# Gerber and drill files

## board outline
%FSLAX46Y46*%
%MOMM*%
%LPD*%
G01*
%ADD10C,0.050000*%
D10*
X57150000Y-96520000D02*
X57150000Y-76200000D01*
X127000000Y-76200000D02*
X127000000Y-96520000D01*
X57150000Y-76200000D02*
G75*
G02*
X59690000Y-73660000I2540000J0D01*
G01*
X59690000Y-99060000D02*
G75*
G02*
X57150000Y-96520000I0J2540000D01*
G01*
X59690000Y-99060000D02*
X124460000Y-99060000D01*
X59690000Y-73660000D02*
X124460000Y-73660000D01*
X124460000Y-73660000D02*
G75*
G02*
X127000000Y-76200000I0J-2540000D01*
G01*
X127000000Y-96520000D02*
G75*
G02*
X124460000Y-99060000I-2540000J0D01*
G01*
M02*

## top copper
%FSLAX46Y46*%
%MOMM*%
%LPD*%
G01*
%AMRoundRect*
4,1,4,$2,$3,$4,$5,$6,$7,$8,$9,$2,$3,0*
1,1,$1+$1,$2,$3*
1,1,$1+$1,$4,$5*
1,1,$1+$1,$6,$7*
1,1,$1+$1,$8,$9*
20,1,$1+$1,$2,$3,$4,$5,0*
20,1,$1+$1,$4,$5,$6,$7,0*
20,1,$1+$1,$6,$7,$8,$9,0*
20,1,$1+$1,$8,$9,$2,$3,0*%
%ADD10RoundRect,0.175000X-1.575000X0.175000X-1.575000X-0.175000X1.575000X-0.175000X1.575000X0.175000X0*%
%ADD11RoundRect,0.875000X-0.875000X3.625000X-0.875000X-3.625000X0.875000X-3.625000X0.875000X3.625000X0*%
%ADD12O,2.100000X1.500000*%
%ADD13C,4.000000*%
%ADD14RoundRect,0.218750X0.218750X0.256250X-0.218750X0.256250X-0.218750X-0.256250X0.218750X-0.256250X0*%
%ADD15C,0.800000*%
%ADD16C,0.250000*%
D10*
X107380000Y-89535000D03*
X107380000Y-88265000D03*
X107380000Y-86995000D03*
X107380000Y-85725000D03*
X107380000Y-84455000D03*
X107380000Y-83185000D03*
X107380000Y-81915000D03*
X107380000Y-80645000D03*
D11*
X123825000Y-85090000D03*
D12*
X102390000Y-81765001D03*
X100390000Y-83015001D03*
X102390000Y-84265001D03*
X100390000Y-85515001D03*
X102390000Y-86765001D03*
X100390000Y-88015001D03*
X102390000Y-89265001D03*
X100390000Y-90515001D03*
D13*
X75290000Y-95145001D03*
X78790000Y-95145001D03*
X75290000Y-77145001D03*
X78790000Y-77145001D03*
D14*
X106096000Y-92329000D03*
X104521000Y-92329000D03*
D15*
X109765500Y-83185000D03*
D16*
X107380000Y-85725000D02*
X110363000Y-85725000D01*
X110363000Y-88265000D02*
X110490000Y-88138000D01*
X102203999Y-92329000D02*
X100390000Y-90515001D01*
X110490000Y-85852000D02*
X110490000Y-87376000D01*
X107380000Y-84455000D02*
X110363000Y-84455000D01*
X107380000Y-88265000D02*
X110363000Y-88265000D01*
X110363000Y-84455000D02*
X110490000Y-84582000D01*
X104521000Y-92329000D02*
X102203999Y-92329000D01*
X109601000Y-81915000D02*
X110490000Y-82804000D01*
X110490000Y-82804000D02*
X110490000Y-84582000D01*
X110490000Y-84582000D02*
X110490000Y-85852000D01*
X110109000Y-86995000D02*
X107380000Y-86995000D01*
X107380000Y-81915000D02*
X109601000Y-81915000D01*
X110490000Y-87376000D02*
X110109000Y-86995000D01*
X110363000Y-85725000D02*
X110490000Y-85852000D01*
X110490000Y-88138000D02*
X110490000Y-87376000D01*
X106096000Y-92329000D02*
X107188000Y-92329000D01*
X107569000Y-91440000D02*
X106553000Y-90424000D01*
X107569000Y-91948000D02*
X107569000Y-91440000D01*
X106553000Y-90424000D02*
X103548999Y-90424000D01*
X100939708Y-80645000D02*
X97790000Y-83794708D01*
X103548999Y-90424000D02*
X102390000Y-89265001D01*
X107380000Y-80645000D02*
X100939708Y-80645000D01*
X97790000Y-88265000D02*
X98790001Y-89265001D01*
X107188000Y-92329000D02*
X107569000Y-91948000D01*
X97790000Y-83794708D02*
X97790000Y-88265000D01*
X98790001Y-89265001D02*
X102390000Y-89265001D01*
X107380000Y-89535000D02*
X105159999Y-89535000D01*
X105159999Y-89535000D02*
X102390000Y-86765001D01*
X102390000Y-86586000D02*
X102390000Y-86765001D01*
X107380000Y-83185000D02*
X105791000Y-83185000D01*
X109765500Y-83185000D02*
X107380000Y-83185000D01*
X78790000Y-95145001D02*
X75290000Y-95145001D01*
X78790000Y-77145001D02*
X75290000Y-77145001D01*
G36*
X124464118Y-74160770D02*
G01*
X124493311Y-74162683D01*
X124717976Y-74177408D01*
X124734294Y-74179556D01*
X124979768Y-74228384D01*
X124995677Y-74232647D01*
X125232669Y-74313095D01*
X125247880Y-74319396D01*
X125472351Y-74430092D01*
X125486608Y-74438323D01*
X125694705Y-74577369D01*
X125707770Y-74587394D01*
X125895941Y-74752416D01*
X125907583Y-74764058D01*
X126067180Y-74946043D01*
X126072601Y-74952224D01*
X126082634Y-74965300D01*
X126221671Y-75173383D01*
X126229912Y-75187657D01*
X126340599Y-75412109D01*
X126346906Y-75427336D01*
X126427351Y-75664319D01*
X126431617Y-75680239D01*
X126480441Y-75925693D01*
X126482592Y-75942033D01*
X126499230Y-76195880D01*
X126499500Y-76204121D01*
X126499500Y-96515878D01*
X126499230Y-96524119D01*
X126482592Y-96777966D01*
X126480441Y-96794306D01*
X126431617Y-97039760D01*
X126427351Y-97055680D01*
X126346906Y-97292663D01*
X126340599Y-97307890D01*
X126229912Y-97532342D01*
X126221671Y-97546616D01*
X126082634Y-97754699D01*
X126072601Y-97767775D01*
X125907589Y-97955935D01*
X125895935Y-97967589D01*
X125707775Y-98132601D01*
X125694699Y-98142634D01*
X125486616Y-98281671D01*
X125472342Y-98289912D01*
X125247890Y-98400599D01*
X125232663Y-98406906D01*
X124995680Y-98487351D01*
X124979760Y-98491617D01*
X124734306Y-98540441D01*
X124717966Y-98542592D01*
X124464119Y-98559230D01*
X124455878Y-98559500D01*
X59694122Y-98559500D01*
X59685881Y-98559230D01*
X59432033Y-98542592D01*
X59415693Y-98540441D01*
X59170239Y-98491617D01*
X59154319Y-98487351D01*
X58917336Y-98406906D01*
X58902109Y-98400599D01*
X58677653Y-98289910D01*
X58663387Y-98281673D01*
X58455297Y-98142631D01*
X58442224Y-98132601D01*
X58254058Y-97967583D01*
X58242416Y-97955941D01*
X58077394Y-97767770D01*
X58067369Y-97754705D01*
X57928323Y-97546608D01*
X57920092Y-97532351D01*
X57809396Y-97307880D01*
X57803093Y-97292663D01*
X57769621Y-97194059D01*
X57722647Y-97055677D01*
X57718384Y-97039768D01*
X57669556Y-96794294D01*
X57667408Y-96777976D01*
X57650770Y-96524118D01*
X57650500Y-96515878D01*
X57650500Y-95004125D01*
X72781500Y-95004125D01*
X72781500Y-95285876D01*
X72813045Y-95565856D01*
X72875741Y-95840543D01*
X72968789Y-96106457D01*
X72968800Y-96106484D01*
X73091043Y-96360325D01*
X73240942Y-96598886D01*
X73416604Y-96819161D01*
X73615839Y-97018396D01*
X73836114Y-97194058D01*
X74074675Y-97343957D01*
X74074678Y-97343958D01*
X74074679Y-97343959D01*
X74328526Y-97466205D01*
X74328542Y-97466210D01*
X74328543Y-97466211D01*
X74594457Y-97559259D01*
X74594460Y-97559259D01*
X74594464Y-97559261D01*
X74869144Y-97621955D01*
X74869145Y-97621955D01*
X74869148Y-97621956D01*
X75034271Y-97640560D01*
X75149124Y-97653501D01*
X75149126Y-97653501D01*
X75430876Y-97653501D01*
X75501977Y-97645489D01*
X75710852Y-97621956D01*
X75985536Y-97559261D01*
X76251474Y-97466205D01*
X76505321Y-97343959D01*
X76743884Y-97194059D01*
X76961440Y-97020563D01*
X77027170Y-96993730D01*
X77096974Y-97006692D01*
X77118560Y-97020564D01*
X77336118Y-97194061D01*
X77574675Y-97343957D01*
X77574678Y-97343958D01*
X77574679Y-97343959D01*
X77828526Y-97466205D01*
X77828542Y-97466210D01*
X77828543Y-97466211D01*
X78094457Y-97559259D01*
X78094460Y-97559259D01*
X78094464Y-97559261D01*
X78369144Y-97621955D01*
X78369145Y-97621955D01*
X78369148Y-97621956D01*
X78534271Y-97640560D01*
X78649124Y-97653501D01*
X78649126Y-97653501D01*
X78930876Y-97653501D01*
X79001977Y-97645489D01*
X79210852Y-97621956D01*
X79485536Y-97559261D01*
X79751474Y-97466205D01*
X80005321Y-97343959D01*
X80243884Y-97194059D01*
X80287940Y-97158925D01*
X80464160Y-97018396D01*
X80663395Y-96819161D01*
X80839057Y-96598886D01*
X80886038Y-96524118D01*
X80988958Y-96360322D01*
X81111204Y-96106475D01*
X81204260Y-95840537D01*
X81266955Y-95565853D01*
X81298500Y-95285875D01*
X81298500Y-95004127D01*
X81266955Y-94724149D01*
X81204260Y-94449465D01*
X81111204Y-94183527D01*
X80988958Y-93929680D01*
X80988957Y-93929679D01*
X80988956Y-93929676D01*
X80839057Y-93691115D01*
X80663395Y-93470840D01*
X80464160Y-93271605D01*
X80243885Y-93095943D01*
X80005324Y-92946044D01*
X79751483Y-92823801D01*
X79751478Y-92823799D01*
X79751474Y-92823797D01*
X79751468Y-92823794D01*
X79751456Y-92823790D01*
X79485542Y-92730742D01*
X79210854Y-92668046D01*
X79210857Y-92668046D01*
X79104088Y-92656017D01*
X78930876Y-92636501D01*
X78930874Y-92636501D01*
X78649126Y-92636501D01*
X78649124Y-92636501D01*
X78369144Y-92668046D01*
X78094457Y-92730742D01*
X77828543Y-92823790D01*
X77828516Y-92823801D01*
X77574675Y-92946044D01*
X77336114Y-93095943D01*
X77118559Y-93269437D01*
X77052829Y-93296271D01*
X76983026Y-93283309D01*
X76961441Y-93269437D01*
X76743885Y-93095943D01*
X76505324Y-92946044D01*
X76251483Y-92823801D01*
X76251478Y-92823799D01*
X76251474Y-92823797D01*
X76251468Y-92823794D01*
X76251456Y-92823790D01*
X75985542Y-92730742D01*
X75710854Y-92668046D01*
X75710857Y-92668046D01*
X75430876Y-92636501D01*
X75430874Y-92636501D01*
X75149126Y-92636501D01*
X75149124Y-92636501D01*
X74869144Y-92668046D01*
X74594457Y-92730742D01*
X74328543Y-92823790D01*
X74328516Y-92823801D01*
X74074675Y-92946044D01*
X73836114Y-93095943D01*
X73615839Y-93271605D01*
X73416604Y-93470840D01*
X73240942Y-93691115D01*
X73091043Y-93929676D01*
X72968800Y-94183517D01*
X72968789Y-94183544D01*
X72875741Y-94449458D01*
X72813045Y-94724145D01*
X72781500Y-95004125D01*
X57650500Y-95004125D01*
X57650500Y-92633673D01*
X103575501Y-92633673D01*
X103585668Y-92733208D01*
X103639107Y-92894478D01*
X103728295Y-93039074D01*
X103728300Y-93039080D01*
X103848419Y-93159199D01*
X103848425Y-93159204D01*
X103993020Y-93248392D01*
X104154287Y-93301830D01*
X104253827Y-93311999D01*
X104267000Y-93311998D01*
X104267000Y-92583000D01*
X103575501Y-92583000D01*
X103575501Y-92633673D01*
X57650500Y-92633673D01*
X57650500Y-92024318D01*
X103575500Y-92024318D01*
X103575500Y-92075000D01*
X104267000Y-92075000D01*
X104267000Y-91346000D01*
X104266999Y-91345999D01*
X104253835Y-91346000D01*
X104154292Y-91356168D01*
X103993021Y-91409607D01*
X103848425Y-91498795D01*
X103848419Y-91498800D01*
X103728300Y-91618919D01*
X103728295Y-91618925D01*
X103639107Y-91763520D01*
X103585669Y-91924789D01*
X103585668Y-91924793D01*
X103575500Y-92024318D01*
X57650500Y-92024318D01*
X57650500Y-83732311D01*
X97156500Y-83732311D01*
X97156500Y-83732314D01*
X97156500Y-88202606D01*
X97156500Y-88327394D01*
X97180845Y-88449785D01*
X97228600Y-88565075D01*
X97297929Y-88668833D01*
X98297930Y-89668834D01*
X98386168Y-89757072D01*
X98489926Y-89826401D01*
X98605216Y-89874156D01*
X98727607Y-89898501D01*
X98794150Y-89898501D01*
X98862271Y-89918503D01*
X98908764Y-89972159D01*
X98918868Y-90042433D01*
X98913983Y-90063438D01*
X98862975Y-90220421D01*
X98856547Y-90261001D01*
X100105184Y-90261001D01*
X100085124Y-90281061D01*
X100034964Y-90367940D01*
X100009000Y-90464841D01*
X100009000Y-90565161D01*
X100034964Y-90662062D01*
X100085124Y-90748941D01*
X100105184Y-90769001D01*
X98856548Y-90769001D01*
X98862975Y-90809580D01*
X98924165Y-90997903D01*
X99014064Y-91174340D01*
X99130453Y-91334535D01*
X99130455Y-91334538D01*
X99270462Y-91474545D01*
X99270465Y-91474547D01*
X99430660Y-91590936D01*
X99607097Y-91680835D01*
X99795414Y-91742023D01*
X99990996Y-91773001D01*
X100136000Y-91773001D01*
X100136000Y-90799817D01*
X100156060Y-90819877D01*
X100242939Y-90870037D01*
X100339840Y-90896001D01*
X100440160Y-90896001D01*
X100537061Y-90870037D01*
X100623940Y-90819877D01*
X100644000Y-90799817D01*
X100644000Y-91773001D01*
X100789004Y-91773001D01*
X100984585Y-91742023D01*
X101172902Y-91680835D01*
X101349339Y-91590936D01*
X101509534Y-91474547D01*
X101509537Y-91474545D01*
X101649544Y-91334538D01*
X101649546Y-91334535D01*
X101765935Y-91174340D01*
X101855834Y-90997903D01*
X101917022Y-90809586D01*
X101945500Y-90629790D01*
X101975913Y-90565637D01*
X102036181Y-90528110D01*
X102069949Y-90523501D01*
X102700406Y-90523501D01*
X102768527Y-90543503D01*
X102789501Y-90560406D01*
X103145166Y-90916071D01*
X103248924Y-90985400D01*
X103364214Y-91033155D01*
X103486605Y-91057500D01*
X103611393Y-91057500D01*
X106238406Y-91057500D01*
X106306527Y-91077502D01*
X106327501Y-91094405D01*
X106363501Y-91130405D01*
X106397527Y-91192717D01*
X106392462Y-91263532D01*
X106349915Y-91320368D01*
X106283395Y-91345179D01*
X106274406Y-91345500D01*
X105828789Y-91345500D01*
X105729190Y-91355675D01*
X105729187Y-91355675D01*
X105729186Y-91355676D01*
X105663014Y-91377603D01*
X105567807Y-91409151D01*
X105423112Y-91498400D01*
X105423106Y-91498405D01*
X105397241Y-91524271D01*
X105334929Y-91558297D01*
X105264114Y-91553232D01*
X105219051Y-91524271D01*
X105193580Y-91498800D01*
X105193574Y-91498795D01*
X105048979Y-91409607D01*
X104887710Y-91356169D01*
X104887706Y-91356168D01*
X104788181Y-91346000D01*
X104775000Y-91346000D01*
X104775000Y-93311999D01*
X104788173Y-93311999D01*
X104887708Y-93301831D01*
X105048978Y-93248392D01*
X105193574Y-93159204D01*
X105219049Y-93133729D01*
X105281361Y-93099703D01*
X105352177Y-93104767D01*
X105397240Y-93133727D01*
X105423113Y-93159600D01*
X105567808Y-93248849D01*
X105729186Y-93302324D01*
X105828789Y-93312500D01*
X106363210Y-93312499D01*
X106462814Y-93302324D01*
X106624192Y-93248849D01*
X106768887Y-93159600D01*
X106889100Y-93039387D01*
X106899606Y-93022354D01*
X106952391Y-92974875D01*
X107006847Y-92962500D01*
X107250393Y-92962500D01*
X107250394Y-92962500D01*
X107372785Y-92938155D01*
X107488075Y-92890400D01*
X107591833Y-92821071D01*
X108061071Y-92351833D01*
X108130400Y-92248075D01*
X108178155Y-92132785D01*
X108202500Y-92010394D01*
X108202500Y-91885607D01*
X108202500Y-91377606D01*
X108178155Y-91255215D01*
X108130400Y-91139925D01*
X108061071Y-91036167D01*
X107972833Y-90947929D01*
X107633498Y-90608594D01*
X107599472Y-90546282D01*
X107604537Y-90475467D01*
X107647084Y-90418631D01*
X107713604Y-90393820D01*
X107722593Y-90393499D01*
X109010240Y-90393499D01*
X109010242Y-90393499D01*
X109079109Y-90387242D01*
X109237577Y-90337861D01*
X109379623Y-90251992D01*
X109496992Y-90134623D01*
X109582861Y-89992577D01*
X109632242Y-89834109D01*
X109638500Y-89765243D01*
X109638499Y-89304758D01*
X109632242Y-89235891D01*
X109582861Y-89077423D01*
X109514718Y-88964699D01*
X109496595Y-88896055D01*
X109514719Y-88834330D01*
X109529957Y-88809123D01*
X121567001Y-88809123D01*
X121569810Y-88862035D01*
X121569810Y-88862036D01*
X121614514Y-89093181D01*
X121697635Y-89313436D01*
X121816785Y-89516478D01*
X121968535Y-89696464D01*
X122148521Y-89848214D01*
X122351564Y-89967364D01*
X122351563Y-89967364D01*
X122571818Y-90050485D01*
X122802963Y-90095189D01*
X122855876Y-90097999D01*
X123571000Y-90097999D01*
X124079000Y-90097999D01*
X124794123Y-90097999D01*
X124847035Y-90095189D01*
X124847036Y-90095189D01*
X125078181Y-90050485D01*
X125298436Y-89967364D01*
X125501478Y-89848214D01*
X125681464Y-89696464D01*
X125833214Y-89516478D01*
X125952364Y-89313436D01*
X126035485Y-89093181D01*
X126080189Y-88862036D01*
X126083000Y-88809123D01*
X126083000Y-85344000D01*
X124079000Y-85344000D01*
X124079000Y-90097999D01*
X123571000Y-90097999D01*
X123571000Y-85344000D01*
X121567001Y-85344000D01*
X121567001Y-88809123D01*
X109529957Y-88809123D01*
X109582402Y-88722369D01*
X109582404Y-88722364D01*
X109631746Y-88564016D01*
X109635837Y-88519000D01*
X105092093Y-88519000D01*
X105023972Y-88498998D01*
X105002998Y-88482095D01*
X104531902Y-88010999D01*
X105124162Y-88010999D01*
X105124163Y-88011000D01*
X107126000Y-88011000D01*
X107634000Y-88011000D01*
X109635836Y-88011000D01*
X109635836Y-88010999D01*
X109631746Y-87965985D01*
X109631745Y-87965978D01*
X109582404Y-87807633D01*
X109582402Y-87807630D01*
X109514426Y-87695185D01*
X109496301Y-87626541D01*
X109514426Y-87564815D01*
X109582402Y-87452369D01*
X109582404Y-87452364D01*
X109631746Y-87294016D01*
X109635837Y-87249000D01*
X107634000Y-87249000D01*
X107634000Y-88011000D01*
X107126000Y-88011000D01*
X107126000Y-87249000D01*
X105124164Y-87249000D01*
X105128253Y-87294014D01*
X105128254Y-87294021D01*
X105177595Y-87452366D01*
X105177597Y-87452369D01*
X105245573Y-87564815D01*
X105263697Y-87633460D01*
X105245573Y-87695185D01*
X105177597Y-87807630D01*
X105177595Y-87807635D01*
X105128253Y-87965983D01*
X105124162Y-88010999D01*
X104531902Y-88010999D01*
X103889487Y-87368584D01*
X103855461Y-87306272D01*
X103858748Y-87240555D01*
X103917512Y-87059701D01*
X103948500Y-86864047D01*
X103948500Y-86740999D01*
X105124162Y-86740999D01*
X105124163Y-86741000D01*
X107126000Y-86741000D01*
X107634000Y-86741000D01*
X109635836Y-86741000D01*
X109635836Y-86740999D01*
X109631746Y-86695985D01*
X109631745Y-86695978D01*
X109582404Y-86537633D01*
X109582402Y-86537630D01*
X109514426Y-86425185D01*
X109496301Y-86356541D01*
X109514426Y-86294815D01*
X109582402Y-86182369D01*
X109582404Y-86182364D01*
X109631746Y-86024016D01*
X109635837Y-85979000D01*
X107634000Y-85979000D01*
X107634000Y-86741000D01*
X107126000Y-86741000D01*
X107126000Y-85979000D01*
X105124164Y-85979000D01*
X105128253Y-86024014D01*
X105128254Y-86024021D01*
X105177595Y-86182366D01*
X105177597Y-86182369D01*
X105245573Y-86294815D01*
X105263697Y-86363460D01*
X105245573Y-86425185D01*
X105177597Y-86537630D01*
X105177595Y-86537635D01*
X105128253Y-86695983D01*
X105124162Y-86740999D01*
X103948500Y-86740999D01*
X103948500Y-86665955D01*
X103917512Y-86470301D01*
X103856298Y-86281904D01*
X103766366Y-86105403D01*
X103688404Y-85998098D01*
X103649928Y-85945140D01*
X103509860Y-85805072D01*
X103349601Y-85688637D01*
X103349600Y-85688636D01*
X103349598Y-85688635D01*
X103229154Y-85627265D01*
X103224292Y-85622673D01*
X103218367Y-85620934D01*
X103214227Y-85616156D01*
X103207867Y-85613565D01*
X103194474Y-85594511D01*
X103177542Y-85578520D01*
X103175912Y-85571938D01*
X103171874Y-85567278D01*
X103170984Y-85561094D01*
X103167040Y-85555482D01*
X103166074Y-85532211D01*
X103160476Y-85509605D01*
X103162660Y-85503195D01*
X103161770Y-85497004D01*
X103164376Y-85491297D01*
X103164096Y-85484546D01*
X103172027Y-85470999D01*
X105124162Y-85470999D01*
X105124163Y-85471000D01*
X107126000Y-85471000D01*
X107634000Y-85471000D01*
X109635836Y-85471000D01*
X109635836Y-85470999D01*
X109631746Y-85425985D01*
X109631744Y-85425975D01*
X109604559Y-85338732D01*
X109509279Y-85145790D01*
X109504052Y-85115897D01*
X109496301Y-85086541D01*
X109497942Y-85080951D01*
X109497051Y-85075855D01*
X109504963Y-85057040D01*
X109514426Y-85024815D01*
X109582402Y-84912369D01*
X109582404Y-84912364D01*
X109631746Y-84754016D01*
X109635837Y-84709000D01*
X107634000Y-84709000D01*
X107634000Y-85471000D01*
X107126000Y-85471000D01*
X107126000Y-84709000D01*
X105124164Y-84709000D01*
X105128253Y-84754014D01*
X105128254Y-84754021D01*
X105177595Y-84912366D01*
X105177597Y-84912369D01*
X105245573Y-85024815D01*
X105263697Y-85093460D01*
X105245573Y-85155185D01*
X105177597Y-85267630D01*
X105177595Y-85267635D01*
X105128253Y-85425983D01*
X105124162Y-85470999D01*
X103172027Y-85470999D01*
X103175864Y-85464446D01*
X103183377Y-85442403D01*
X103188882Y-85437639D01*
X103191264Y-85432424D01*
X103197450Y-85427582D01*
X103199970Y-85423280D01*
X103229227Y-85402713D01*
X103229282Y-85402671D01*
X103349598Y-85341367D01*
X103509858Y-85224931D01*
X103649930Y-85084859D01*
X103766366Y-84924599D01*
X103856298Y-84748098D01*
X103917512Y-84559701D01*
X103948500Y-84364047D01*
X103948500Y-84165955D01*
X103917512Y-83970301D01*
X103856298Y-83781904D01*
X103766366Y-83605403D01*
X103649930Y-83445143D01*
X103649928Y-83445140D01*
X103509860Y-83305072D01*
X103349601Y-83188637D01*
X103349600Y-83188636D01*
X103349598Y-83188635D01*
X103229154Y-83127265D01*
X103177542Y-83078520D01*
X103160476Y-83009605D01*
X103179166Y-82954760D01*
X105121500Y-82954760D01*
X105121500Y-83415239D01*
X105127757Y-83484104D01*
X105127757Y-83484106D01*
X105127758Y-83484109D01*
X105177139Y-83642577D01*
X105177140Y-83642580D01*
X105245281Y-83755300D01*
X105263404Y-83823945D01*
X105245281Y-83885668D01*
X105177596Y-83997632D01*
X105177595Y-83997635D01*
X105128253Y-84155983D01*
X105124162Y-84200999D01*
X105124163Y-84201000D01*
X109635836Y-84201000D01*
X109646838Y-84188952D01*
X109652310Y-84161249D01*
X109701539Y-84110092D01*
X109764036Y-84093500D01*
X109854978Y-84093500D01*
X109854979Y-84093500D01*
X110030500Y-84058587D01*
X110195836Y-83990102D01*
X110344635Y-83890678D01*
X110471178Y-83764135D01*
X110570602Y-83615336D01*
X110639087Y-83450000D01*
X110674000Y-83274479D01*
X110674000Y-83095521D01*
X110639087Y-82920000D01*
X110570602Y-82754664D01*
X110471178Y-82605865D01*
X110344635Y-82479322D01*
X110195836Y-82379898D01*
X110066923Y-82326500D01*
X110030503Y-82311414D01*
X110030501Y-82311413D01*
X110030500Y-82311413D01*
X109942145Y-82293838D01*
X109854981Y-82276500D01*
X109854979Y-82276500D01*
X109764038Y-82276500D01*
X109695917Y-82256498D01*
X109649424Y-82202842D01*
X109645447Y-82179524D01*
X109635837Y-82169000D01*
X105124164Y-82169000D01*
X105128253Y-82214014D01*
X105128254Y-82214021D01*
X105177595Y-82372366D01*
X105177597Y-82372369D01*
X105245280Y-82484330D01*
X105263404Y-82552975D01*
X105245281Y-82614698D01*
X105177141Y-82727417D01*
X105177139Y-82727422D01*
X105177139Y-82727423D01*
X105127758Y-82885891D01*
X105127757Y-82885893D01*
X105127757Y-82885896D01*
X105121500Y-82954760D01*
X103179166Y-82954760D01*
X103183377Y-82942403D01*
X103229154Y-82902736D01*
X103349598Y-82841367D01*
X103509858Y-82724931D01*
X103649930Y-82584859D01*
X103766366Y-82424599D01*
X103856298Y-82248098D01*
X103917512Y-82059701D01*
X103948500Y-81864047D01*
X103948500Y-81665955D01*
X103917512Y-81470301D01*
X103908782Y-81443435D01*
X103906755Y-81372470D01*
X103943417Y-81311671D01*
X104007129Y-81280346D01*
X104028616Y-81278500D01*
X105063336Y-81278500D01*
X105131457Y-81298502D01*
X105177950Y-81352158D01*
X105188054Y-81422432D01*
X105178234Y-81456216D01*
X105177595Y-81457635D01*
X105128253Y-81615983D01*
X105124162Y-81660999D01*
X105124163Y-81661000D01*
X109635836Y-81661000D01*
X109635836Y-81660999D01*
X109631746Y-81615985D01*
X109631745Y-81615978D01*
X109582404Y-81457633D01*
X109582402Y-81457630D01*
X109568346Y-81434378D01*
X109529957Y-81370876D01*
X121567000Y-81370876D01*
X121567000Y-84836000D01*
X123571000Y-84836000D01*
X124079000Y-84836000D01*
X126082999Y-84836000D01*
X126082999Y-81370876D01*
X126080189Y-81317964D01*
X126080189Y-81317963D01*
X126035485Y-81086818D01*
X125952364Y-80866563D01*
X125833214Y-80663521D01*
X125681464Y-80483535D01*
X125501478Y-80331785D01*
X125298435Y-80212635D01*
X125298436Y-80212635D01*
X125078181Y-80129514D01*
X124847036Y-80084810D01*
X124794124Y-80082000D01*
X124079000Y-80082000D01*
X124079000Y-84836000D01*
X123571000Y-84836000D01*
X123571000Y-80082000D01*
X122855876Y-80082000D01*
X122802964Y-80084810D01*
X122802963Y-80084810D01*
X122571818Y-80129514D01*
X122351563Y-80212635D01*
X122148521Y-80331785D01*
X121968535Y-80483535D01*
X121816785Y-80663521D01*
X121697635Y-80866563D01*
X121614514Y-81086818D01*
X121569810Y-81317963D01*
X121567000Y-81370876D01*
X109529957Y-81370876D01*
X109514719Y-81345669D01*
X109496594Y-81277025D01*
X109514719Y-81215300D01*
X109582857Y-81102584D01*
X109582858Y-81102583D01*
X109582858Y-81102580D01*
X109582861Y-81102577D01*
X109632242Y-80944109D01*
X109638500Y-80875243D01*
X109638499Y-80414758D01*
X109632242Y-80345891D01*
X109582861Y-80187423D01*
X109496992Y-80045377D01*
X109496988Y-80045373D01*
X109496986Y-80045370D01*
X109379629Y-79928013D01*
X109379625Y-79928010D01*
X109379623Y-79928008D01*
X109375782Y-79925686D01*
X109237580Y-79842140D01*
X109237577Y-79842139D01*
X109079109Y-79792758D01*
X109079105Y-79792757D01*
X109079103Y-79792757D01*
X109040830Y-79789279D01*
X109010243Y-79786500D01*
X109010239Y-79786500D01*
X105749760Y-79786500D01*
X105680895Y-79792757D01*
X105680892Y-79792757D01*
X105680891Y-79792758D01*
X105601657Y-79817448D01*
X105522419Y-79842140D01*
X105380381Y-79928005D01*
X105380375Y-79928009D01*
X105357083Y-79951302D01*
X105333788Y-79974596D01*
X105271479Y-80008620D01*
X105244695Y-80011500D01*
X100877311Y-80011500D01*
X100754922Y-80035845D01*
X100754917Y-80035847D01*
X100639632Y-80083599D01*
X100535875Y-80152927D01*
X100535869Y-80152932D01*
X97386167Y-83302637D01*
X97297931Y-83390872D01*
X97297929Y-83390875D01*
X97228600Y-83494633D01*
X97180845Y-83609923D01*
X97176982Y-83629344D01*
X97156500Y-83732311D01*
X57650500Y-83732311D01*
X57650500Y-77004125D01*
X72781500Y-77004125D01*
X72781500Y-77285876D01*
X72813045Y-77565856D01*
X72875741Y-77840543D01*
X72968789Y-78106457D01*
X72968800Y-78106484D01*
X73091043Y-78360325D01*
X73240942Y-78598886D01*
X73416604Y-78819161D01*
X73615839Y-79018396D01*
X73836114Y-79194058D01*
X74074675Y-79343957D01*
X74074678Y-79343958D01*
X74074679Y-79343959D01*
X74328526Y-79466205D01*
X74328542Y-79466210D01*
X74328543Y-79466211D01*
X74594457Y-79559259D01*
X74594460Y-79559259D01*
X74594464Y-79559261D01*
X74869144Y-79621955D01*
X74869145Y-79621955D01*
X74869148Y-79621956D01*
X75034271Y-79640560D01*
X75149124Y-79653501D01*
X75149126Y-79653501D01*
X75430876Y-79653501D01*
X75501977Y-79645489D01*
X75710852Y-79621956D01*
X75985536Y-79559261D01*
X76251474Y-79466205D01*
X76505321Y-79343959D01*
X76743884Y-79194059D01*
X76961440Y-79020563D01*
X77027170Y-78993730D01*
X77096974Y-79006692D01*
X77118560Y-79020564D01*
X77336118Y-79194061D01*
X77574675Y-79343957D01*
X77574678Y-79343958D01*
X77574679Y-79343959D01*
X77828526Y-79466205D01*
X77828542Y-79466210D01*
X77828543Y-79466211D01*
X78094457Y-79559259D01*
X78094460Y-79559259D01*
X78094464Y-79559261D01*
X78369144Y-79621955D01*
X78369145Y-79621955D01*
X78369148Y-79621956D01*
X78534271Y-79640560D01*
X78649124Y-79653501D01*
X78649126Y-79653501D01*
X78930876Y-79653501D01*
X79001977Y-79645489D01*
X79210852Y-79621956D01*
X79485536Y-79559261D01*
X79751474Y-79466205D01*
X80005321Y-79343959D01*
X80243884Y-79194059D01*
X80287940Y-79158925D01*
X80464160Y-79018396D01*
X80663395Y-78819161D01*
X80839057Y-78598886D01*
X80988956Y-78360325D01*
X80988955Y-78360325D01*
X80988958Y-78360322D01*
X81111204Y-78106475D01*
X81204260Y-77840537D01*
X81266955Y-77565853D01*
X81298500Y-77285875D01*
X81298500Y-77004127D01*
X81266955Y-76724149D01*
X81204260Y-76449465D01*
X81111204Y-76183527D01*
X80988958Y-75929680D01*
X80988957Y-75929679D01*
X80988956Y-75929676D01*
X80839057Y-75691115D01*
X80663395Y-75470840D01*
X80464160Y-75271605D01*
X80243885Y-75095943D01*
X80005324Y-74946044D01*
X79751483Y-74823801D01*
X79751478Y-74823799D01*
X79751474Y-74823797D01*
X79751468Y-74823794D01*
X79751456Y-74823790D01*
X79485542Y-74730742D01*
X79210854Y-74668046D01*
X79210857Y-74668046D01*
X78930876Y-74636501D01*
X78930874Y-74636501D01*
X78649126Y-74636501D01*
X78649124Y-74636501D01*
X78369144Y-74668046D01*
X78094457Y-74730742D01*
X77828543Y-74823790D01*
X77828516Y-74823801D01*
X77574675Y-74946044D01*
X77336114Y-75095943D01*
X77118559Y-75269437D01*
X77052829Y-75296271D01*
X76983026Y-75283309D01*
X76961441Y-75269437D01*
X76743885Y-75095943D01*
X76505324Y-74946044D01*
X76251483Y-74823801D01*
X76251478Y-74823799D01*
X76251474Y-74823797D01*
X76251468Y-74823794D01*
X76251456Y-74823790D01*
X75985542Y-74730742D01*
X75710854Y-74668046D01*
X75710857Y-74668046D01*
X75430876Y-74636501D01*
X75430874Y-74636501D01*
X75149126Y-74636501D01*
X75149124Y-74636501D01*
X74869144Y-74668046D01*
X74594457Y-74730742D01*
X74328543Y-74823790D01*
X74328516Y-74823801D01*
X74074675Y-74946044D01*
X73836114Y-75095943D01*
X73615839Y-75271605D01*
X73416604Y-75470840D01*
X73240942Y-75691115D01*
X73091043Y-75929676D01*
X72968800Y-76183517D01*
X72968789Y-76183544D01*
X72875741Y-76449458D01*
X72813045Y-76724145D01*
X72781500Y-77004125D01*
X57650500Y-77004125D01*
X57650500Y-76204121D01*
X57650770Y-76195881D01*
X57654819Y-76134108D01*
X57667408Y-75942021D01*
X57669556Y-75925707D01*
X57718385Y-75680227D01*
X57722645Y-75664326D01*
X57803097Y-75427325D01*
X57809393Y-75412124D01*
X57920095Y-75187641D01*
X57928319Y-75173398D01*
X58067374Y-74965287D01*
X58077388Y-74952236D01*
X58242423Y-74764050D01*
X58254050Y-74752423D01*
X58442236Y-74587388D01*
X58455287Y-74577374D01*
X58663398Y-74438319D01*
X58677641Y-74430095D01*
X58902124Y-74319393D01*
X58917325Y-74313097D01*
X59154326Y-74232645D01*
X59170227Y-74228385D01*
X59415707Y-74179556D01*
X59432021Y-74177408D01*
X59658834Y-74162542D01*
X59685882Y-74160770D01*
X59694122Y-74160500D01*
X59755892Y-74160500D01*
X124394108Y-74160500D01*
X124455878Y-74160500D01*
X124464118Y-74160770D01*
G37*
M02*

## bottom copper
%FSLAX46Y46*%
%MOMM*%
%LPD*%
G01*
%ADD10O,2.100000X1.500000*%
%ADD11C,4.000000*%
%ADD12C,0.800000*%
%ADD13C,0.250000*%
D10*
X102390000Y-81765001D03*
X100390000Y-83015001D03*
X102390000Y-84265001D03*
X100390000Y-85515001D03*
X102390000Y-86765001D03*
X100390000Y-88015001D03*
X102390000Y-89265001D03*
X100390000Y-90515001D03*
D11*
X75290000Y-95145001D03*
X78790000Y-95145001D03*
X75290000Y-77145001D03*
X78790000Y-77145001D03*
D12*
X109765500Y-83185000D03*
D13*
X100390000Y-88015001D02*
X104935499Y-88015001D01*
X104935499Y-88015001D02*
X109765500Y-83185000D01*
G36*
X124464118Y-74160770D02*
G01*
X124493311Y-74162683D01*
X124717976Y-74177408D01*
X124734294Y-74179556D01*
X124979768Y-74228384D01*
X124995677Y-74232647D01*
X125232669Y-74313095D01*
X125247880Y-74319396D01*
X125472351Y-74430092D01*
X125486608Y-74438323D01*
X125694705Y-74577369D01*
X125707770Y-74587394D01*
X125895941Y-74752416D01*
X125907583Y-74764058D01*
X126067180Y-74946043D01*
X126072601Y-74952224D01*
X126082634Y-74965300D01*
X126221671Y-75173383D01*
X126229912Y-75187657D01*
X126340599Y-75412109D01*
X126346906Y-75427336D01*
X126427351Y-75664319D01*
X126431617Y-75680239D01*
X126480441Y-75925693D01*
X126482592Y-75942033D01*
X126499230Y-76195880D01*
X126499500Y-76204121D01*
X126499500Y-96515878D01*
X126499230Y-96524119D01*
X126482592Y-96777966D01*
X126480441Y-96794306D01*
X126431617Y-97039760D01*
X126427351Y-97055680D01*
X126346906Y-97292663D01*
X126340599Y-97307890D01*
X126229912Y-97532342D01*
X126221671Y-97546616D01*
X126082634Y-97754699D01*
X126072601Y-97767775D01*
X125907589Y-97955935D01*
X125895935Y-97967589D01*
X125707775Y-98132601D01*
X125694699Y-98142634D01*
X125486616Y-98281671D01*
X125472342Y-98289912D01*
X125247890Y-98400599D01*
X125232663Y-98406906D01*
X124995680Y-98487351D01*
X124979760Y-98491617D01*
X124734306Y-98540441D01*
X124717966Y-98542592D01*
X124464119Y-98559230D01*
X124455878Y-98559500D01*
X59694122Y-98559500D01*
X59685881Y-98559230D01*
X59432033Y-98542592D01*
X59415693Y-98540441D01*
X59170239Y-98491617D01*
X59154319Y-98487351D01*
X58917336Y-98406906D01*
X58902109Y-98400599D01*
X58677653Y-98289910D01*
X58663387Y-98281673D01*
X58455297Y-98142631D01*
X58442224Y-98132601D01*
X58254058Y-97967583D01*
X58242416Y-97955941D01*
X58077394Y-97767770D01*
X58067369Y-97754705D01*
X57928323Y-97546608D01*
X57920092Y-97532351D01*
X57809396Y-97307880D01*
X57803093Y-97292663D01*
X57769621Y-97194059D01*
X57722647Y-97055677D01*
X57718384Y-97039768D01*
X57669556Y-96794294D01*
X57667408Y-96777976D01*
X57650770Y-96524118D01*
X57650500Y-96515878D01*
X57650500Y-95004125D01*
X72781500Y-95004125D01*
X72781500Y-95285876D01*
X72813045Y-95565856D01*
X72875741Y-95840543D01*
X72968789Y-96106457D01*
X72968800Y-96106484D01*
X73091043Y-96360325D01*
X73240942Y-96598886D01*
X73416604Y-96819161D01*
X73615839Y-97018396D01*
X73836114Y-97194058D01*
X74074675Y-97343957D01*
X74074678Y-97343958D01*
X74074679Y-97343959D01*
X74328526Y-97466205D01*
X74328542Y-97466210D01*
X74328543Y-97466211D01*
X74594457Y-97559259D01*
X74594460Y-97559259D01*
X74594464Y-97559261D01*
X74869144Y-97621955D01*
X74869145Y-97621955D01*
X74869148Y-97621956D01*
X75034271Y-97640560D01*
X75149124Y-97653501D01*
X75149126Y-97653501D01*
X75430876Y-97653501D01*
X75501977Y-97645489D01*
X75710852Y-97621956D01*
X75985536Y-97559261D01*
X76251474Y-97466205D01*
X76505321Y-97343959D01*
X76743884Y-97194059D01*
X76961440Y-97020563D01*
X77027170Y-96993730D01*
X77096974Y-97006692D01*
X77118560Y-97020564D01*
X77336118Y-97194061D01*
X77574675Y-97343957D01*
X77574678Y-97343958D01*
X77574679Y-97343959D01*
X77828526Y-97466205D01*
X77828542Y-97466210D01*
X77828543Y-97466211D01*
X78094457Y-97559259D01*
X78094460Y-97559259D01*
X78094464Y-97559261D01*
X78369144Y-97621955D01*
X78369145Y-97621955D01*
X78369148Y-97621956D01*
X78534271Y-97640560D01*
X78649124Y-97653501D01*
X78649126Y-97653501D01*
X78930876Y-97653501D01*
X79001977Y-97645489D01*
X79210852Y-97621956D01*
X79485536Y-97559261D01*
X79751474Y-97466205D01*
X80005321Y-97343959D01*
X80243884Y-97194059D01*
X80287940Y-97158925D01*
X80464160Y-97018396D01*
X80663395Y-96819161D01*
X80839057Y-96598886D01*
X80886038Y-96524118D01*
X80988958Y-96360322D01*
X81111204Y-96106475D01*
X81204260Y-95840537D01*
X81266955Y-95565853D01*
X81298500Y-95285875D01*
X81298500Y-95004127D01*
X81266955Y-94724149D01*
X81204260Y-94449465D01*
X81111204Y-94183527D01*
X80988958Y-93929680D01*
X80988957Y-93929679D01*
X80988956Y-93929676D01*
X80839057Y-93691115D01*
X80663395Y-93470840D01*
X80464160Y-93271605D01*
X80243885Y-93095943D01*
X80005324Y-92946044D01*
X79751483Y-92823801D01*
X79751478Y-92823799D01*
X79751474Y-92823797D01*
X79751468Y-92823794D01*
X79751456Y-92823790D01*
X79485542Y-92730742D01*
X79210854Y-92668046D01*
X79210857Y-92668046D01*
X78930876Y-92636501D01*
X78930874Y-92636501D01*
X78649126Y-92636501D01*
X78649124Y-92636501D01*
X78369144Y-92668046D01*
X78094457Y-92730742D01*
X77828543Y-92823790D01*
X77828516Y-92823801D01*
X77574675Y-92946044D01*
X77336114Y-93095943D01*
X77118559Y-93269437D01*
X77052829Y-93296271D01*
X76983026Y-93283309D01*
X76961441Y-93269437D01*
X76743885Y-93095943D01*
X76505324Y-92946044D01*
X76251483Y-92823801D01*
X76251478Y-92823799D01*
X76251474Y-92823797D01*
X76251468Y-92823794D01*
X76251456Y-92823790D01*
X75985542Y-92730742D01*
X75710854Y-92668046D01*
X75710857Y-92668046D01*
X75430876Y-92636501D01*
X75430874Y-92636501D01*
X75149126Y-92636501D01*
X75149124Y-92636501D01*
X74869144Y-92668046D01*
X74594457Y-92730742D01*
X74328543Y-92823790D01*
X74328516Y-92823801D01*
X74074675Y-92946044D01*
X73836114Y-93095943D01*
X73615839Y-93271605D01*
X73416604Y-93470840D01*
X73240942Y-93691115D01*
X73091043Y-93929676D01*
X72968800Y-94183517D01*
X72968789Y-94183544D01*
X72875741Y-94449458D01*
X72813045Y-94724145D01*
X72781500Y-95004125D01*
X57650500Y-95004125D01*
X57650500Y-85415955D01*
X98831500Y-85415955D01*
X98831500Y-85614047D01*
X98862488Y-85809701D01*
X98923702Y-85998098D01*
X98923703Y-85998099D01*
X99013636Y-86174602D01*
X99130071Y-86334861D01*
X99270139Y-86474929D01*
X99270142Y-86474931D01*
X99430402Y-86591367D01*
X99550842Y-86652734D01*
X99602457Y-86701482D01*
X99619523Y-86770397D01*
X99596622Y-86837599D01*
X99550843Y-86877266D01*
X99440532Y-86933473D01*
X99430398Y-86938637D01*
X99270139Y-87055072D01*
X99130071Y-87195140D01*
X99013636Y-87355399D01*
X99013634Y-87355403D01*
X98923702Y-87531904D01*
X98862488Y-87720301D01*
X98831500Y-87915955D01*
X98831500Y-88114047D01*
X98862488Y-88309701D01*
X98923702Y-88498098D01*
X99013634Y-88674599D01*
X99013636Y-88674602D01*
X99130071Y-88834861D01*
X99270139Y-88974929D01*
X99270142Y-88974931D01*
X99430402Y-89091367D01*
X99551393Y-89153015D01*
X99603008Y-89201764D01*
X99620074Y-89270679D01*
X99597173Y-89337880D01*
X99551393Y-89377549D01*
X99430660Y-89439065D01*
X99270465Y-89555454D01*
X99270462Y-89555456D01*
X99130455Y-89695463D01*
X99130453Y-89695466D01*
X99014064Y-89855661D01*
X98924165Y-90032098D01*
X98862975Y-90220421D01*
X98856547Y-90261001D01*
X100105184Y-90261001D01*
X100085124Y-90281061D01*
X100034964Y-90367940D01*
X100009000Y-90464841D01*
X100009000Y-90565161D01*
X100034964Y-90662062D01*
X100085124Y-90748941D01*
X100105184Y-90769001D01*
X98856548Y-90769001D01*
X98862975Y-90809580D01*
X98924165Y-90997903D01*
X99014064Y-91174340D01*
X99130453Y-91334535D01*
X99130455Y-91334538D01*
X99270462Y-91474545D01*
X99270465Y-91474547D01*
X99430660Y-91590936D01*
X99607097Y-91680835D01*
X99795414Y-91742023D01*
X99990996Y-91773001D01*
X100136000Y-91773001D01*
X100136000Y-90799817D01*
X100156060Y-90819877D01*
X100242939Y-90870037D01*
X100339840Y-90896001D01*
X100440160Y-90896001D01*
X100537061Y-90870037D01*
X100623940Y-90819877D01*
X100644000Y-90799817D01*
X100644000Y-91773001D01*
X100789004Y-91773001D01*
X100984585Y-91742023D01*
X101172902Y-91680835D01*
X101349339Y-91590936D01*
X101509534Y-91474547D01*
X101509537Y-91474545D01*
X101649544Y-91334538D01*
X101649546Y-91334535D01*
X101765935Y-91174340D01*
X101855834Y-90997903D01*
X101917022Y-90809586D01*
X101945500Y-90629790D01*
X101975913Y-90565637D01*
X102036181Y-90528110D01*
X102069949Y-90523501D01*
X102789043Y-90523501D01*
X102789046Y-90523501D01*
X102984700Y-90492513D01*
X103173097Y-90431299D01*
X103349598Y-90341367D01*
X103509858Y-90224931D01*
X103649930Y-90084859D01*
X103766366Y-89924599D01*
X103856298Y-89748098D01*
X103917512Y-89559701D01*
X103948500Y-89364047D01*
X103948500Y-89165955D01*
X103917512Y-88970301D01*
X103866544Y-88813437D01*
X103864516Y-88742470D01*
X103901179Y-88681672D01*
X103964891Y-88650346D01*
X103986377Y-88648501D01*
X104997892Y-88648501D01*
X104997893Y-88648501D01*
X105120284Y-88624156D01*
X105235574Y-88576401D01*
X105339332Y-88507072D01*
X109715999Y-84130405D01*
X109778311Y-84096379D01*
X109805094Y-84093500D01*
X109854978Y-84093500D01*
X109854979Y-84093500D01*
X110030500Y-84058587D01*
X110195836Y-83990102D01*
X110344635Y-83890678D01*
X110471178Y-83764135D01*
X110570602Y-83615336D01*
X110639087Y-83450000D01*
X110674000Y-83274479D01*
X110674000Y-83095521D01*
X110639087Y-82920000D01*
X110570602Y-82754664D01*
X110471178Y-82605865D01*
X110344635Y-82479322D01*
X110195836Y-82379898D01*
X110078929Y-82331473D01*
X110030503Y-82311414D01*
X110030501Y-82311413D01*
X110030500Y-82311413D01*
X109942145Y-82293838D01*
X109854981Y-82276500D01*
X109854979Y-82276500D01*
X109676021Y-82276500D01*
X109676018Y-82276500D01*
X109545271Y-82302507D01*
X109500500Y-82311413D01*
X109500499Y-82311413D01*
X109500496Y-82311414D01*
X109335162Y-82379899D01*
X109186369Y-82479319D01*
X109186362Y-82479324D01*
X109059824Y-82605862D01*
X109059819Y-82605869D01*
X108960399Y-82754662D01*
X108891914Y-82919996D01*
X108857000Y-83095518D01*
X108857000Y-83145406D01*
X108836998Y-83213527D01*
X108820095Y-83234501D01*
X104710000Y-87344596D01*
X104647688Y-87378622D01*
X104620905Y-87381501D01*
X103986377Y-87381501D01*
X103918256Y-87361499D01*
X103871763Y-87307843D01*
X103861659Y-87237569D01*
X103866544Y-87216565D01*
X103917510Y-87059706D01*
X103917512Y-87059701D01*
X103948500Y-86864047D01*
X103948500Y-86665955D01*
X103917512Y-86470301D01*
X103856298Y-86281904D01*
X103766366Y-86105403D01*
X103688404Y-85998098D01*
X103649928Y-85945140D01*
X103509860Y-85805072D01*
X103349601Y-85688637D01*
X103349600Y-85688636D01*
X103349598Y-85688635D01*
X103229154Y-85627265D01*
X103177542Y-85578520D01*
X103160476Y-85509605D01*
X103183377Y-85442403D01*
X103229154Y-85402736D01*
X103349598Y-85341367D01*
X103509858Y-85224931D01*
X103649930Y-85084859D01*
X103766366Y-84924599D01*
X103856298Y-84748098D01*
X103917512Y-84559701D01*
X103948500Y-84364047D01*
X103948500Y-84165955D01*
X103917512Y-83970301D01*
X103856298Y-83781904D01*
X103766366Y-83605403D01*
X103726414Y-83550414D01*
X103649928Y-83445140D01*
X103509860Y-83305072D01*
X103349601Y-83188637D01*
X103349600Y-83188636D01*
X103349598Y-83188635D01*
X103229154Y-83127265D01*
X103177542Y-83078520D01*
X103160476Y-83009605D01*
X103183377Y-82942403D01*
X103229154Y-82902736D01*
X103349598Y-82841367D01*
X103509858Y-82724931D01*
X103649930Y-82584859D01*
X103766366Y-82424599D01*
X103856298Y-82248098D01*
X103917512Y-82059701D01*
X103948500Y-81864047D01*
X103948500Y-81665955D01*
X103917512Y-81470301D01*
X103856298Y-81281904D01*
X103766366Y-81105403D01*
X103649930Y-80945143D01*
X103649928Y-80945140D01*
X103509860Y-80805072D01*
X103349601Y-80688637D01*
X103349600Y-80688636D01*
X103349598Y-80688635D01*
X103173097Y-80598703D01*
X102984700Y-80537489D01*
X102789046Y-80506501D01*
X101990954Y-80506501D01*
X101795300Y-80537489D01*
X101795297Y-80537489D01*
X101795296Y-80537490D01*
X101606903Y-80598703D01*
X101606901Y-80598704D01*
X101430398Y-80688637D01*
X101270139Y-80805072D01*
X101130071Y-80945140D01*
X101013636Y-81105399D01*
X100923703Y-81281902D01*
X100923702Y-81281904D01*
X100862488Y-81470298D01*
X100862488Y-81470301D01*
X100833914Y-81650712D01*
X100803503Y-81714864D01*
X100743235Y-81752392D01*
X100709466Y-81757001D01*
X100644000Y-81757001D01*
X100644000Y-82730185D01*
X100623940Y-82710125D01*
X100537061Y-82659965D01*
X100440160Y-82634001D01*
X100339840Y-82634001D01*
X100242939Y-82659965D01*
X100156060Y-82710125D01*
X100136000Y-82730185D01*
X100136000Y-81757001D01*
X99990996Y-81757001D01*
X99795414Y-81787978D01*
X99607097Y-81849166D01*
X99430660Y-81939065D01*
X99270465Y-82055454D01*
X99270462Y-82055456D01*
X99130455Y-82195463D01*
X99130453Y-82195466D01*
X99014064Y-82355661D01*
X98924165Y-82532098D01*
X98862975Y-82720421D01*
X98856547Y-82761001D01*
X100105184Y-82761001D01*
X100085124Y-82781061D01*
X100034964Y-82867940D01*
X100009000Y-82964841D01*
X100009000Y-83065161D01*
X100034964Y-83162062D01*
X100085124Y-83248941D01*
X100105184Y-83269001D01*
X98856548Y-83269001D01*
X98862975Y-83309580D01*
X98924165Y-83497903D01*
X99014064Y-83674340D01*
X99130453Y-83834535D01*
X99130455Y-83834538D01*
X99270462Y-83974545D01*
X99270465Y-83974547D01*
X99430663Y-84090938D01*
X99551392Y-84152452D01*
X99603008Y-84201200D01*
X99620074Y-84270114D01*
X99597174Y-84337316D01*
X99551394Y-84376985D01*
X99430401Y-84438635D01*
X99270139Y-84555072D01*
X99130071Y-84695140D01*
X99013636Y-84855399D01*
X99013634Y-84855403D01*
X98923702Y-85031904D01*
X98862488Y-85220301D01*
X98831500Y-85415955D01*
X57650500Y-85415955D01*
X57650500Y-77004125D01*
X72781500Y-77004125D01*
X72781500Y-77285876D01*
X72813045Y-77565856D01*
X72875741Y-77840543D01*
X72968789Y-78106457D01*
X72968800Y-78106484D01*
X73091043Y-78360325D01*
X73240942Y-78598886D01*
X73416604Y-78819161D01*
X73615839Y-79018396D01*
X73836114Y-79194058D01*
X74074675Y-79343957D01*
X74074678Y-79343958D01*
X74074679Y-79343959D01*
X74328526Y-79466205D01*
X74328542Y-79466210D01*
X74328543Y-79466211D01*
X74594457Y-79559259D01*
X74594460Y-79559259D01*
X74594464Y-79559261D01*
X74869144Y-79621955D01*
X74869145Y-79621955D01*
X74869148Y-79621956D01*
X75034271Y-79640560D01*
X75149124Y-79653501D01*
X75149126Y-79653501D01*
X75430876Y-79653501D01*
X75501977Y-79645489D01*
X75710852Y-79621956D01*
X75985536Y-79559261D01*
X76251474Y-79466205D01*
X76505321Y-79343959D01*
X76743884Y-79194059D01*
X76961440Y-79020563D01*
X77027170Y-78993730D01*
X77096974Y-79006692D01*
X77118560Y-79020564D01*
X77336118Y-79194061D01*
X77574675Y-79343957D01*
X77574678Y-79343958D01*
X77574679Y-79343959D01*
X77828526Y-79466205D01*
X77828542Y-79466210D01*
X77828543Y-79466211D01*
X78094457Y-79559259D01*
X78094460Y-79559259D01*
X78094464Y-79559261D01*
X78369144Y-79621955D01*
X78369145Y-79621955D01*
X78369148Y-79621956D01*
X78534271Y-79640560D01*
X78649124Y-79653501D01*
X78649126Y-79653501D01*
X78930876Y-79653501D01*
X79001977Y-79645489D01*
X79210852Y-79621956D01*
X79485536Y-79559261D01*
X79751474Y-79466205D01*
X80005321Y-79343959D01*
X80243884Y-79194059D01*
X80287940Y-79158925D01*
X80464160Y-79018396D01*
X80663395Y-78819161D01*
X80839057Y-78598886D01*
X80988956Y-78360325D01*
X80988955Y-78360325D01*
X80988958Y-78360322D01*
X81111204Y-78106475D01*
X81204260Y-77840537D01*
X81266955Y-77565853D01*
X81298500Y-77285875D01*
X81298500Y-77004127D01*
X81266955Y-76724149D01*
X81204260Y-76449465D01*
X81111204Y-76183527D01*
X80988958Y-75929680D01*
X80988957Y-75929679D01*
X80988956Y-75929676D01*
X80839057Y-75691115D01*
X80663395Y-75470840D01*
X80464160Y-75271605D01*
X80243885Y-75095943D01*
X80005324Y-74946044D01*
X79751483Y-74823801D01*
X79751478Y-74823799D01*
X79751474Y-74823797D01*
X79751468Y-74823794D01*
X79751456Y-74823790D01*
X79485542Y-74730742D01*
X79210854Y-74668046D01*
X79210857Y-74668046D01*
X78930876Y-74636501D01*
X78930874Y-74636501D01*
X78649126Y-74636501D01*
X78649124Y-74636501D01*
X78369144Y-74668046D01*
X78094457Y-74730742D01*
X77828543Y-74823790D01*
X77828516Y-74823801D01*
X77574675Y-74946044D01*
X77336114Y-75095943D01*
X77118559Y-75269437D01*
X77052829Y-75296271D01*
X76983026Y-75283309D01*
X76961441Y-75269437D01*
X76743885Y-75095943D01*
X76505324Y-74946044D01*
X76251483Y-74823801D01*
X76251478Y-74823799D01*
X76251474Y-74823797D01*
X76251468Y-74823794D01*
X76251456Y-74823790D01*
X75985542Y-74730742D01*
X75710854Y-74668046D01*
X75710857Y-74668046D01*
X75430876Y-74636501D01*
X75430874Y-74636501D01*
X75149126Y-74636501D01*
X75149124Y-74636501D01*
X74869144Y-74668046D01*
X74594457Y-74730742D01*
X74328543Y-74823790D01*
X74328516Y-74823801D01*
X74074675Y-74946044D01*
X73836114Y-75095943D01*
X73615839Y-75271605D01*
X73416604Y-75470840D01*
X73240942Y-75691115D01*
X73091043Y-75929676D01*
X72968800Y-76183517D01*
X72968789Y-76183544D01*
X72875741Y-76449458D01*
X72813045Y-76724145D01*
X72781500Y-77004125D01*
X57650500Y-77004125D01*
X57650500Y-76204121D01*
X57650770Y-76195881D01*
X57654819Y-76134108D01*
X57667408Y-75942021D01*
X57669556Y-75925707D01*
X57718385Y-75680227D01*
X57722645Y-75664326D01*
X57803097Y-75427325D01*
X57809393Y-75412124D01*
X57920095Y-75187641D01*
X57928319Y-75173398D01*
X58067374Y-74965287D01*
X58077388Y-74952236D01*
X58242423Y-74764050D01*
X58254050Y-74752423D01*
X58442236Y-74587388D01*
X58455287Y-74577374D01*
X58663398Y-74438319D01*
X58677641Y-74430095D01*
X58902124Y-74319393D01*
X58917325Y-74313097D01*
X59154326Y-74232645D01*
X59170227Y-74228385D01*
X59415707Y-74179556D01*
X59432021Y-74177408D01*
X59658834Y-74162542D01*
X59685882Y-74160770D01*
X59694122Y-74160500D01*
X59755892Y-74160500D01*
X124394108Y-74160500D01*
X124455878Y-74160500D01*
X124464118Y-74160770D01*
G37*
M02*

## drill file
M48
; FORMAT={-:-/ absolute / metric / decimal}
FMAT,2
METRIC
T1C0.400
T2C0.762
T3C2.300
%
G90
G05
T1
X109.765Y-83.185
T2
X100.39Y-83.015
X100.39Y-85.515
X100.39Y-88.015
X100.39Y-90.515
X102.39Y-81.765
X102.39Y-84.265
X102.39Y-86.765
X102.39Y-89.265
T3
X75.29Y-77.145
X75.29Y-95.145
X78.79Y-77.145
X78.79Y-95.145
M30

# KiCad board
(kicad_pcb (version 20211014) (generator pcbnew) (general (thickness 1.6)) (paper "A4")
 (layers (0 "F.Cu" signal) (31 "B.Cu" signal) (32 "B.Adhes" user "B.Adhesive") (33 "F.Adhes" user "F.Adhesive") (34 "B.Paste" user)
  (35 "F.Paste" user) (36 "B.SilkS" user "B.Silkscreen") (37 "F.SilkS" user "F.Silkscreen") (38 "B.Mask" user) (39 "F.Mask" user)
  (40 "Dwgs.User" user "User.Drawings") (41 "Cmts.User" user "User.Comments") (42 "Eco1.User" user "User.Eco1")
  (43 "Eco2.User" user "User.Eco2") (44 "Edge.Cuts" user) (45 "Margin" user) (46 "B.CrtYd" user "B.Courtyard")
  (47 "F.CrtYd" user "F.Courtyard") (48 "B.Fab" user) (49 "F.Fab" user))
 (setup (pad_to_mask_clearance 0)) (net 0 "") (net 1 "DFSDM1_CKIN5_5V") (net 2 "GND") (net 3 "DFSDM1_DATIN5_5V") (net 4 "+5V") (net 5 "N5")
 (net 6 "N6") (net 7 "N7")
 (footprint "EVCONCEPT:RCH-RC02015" (layer "F.Cu") (at 115.57 85.09 -90)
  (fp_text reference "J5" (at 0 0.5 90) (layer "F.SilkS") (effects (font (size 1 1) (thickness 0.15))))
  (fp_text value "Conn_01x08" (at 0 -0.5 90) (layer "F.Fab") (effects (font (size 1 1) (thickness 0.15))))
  (pad "1" smd roundrect locked (at 4.445 8.19 270) (size 0.7 3.5) (layers "F.Cu" "F.Paste" "F.Mask") (roundrect_rratio 0.25)
   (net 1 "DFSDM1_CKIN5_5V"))
  (pad "2" smd roundrect locked (at 3.175 8.19 270) (size 0.7 3.5) (layers "F.Cu" "F.Paste" "F.Mask") (roundrect_rratio 0.25) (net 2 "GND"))
  (pad "3" smd roundrect locked (at 1.905 8.19 270) (size 0.7 3.5) (layers "F.Cu" "F.Paste" "F.Mask") (roundrect_rratio 0.25) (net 2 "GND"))
  (pad "4" smd roundrect locked (at 0.635 8.19 270) (size 0.7 3.5) (layers "F.Cu" "F.Paste" "F.Mask") (roundrect_rratio 0.25) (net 2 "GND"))
  (pad "5" smd roundrect locked (at -0.635 8.19 270) (size 0.7 3.5) (layers "F.Cu" "F.Paste" "F.Mask") (roundrect_rratio 0.25) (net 2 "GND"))
  (pad "6" smd roundrect locked (at -1.905 8.19 270) (size 0.7 3.5) (layers "F.Cu" "F.Paste" "F.Mask") (roundrect_rratio 0.25)
   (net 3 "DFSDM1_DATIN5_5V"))
  (pad "7" smd roundrect locked (at -3.175 8.19 270) (size 0.7 3.5) (layers "F.Cu" "F.Paste" "F.Mask") (roundrect_rratio 0.25) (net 2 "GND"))
  (pad "8" smd roundrect locked (at -4.445 8.19 270) (size 0.7 3.5) (layers "F.Cu" "F.Paste" "F.Mask") (roundrect_rratio 0.25) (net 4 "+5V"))
  (pad "9" smd roundrect locked (at 0 -8.255 270) (size 9 3.5) (layers "F.Cu" "F.Paste" "F.Mask") (roundrect_rratio 0.25) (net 2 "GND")))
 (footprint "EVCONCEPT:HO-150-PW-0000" (layer "F.Cu") (at 100.39 86.145001)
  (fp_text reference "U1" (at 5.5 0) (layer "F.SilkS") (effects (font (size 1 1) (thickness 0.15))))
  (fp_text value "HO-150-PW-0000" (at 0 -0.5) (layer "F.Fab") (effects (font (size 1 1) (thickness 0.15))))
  (pad "1" thru_hole oval locked (at 2 -4.38) (size 2.1 1.5) (drill 0.762) (layers *.Cu *.Mask) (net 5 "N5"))
  (pad "2" thru_hole oval locked (at 0 -3.13) (size 2.1 1.5) (drill 0.762) (layers *.Cu *.Mask) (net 2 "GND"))
  (pad "3" thru_hole oval locked (at 2 -1.88) (size 2.1 1.5) (drill 0.762) (layers *.Cu *.Mask))
  (pad "4" thru_hole oval locked (at 0 -0.63) (size 2.1 1.5) (drill 0.762) (layers *.Cu *.Mask))
  (pad "5" thru_hole oval locked (at 2 0.62) (size 2.1 1.5) (drill 0.762) (layers *.Cu *.Mask) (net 1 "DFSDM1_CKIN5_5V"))
  (pad "6" thru_hole oval locked (at 0 1.87) (size 2.1 1.5) (drill 0.762) (layers *.Cu *.Mask) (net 3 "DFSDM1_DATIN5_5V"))
  (pad "7" thru_hole oval locked (at 2 3.12) (size 2.1 1.5) (drill 0.762) (layers *.Cu *.Mask) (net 4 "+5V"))
  (pad "8" thru_hole oval locked (at 0 4.37) (size 2.1 1.5) (drill 0.762) (layers *.Cu *.Mask) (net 2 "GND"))
  (pad "9" thru_hole circle locked (at -25.1 9) (size 4 4) (drill 2.3) (layers *.Cu *.Mask) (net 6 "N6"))
  (pad "9" thru_hole circle locked (at -21.6 9) (size 4 4) (drill 2.3) (layers *.Cu *.Mask) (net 6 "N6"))
  (pad "10" thru_hole circle locked (at -25.1 -9) (size 4 4) (drill 2.3) (layers *.Cu *.Mask) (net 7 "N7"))
  (pad "10" thru_hole circle locked (at -21.6 -9) (size 4 4) (drill 2.3) (layers *.Cu *.Mask) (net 7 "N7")))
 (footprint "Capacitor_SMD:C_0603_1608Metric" (layer "F.Cu") (at 105.3085 92.329 180)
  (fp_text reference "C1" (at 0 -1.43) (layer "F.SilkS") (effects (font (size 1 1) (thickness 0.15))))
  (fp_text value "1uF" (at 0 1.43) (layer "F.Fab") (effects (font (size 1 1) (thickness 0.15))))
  (pad "1" smd roundrect locked (at -0.7875 0 180) (size 0.875 0.95) (layers "F.Cu" "F.Paste" "F.Mask") (roundrect_rratio 0.25)
   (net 4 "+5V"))
  (pad "2" smd roundrect locked (at 0.7875 0 180) (size 0.875 0.95) (layers "F.Cu" "F.Paste" "F.Mask") (roundrect_rratio 0.25) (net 2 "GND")))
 (gr_line (start 57.15 96.52) (end 57.15 76.2) (layer "Edge.Cuts") (width 0.05))
 (gr_line (start 127 76.2) (end 127 96.52) (layer "Edge.Cuts") (width 0.05))
 (gr_arc (start 57.15 76.2) (mid 57.893949 74.403949) (end 59.69 73.66) (layer "Edge.Cuts") (width 0.05))
 (gr_arc (start 59.69 99.06) (mid 57.893949 98.316051) (end 57.15 96.52) (layer "Edge.Cuts") (width 0.05))
 (gr_line (start 59.69 99.06) (end 124.46 99.06) (layer "Edge.Cuts") (width 0.05))
 (gr_line (start 59.69 73.66) (end 124.46 73.66) (layer "Edge.Cuts") (width 0.05))
 (gr_arc (start 124.46 73.66) (mid 126.256051 74.403949) (end 127 76.2) (layer "Edge.Cuts") (width 0.05))
 (gr_arc (start 127 96.52) (mid 126.256051 98.316051) (end 124.46 99.06) (layer "Edge.Cuts") (width 0.05))
 (segment (start 107.38 85.725) (end 110.363 85.725) (width 0.25) (layer "F.Cu") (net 2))
 (segment (start 110.363 88.265) (end 110.49 88.138) (width 0.25) (layer "F.Cu") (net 2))
 (segment (start 102.203999 92.329) (end 100.39 90.515001) (width 0.25) (layer "F.Cu") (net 2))
 (segment (start 110.49 85.852) (end 110.49 87.376) (width 0.25) (layer "F.Cu") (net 2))
 (segment (start 107.38 84.455) (end 110.363 84.455) (width 0.25) (layer "F.Cu") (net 2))
 (segment (start 107.38 88.265) (end 110.363 88.265) (width 0.25) (layer "F.Cu") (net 2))
 (segment (start 110.363 84.455) (end 110.49 84.582) (width 0.25) (layer "F.Cu") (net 2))
 (segment (start 104.521 92.329) (end 102.203999 92.329) (width 0.25) (layer "F.Cu") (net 2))
 (segment (start 109.601 81.915) (end 110.49 82.804) (width 0.25) (layer "F.Cu") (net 2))
 (segment (start 110.49 82.804) (end 110.49 84.582) (width 0.25) (layer "F.Cu") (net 2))
 (segment (start 110.49 84.582) (end 110.49 85.852) (width 0.25) (layer "F.Cu") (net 2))
 (segment (start 110.109 86.995) (end 107.38 86.995) (width 0.25) (layer "F.Cu") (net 2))
 (segment (start 107.38 81.915) (end 109.601 81.915) (width 0.25) (layer "F.Cu") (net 2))
 (segment (start 110.49 87.376) (end 110.109 86.995) (width 0.25) (layer "F.Cu") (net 2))
 (segment (start 110.363 85.725) (end 110.49 85.852) (width 0.25) (layer "F.Cu") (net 2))
 (segment (start 110.49 88.138) (end 110.49 87.376) (width 0.25) (layer "F.Cu") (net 2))
 (segment (start 106.096 92.329) (end 107.188 92.329) (width 0.25) (layer "F.Cu") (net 4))
 (segment (start 107.569 91.44) (end 106.553 90.424) (width 0.25) (layer "F.Cu") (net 4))
 (segment (start 107.569 91.948) (end 107.569 91.44) (width 0.25) (layer "F.Cu") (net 4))
 (segment (start 106.553 90.424) (end 103.548999 90.424) (width 0.25) (layer "F.Cu") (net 4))
 (segment (start 100.939708 80.645) (end 97.79 83.794708) (width 0.25) (layer "F.Cu") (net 4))
 (segment (start 103.548999 90.424) (end 102.39 89.265001) (width 0.25) (layer "F.Cu") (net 4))
 (segment (start 107.38 80.645) (end 100.939708 80.645) (width 0.25) (layer "F.Cu") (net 4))
 (segment (start 97.79 88.265) (end 98.790001 89.265001) (width 0.25) (layer "F.Cu") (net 4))
 (segment (start 107.188 92.329) (end 107.569 91.948) (width 0.25) (layer "F.Cu") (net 4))
 (segment (start 97.79 83.794708) (end 97.79 88.265) (width 0.25) (layer "F.Cu") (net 4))
 (segment (start 98.790001 89.265001) (end 102.39 89.265001) (width 0.25) (layer "F.Cu") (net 4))
 (segment (start 107.38 89.535) (end 105.159999 89.535) (width 0.25) (layer "F.Cu") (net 1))
 (segment (start 105.159999 89.535) (end 102.39 86.765001) (width 0.25) (layer "F.Cu") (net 1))
 (segment (start 102.39 86.586) (end 102.39 86.765001) (width 0.25) (layer "F.Cu") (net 1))
 (segment (start 107.38 83.185) (end 105.791 83.185) (width 0.25) (layer "F.Cu") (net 3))
 (segment (start 109.7655 83.185) (end 107.38 83.185) (width 0.25) (layer "F.Cu") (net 3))
 (via (at 109.7655 83.185) (size 0.8) (drill 0.4) (layers "F.Cu" "B.Cu") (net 3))
 (segment (start 100.39 88.015001) (end 104.935499 88.015001) (width 0.25) (layer "B.Cu") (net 3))
 (segment (start 104.935499 88.015001) (end 109.7655 83.185) (width 0.25) (layer "B.Cu") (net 3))
 (segment (start 78.79 95.145001) (end 75.29 95.145001) (width 0.25) (layer "F.Cu") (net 6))
 (segment (start 78.79 77.145001) (end 75.29 77.145001) (width 0.25) (layer "F.Cu") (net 7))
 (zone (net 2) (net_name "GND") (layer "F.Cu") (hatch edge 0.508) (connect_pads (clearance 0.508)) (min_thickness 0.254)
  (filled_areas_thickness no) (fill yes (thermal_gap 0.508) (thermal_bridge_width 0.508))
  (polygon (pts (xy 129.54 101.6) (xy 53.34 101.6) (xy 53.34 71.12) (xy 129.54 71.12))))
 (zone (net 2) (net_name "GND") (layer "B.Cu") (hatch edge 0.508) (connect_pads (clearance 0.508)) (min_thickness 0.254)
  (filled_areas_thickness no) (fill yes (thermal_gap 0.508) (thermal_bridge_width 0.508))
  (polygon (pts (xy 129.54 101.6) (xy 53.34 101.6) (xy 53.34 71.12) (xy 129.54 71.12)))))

